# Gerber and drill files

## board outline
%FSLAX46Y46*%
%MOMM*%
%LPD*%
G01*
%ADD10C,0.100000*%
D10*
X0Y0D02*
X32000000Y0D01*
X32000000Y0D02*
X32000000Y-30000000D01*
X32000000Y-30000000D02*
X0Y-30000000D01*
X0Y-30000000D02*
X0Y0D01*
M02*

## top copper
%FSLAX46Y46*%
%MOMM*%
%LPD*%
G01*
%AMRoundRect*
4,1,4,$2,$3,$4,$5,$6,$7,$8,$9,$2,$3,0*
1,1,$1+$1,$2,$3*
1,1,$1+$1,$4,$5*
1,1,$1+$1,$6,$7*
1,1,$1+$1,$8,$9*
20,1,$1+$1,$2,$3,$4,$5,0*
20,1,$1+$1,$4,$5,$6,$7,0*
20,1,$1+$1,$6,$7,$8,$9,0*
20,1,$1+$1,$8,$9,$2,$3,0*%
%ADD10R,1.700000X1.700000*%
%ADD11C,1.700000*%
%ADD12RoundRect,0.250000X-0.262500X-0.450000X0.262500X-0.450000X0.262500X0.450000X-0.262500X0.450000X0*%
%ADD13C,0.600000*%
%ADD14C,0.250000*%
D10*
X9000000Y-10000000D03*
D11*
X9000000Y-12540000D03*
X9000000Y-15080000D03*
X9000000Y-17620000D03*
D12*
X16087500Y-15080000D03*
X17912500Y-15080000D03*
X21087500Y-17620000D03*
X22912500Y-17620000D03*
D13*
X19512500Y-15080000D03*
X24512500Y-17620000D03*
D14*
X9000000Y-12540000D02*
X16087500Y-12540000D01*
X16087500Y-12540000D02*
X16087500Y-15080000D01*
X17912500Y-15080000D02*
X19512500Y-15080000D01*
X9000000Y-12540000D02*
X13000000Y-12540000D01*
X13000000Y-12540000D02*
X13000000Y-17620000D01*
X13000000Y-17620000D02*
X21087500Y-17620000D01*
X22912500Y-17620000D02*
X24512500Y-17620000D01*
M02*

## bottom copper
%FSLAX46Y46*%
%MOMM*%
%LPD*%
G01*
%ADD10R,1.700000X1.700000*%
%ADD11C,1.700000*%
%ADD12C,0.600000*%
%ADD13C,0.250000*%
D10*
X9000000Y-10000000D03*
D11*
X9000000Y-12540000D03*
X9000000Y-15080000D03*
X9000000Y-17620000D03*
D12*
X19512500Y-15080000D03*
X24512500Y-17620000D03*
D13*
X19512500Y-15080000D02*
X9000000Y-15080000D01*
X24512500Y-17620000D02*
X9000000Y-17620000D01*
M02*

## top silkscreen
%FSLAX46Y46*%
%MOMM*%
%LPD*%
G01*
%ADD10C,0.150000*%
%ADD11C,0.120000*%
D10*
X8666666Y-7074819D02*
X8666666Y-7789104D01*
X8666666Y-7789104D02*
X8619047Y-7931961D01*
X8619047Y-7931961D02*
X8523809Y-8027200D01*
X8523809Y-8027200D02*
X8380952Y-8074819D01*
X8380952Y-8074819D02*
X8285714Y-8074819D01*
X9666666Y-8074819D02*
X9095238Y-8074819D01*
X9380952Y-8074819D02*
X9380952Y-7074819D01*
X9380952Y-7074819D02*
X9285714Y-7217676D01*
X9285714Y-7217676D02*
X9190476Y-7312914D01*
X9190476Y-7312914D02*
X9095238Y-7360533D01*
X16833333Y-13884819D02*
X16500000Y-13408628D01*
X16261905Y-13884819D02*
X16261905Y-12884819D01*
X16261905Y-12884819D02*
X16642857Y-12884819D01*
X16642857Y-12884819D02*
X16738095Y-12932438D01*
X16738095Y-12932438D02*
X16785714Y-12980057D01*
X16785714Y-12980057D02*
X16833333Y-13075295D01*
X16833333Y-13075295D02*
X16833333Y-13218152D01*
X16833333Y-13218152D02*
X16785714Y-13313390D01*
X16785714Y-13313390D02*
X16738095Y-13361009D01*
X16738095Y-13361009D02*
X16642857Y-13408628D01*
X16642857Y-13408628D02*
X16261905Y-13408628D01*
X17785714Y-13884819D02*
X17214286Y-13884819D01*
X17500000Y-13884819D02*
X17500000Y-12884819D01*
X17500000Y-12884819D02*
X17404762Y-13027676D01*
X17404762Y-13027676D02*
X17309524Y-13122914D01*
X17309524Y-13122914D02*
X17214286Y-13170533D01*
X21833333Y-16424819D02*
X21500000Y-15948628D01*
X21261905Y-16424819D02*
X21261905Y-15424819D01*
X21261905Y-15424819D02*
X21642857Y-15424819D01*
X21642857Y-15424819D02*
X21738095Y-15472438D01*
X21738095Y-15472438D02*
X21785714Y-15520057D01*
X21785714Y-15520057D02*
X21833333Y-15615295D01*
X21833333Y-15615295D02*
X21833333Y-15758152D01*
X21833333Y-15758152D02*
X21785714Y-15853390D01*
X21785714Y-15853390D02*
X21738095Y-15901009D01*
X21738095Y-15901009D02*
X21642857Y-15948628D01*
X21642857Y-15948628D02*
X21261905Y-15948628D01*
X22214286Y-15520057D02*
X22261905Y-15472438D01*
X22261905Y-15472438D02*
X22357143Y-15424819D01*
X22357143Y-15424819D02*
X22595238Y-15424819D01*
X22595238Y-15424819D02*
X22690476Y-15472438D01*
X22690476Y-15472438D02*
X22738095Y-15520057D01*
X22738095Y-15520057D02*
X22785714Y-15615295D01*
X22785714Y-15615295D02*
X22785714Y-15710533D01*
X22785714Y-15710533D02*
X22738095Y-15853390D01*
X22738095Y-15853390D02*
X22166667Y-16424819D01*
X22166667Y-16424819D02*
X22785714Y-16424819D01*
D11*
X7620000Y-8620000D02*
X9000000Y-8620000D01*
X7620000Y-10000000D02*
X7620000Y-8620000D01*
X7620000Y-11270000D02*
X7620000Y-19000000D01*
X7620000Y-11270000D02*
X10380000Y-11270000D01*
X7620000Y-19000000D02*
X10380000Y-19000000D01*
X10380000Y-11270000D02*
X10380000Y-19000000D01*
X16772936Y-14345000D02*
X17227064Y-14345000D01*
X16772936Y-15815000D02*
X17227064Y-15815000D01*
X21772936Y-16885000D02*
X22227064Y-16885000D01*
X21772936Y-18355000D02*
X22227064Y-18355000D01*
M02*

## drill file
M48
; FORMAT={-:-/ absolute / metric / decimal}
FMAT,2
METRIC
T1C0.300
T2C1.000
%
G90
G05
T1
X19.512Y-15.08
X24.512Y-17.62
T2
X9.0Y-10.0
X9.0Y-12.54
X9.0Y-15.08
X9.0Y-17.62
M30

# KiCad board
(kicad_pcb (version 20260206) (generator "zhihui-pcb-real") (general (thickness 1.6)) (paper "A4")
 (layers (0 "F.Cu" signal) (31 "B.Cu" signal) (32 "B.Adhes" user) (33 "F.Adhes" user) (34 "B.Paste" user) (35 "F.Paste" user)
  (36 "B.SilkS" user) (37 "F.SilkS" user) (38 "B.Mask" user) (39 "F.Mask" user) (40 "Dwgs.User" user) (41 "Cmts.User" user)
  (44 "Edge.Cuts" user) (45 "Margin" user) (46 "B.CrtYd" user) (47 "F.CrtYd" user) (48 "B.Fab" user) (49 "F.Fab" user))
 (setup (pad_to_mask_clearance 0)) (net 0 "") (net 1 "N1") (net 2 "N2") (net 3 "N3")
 (gr_line (start 0 0) (end 32 0) (stroke (width 0.1) (type default)) (layer "Edge.Cuts"))
 (gr_line (start 32 0) (end 32 30) (stroke (width 0.1) (type default)) (layer "Edge.Cuts"))
 (gr_line (start 32 30) (end 0 30) (stroke (width 0.1) (type default)) (layer "Edge.Cuts"))
 (gr_line (start 0 30) (end 0 0) (stroke (width 0.1) (type default)) (layer "Edge.Cuts"))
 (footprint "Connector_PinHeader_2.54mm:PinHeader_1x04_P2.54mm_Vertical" (layer "F.Cu")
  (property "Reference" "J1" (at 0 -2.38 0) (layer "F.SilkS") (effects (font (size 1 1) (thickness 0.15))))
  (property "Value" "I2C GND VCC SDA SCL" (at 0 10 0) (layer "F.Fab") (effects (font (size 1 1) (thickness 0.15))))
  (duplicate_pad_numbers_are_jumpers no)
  (fp_line (start -1.38 -1.38) (end 0 -1.38) (stroke (width 0.12) (type solid)) (layer "F.SilkS"))
  (fp_line (start -1.38 0) (end -1.38 -1.38) (stroke (width 0.12) (type solid)) (layer "F.SilkS"))
  (fp_line (start -1.38 1.27) (end -1.38 9) (stroke (width 0.12) (type solid)) (layer "F.SilkS"))
  (fp_line (start -1.38 1.27) (end 1.38 1.27) (stroke (width 0.12) (type solid)) (layer "F.SilkS"))
  (fp_line (start -1.38 9) (end 1.38 9) (stroke (width 0.12) (type solid)) (layer "F.SilkS"))
  (fp_line (start 1.38 1.27) (end 1.38 9) (stroke (width 0.12) (type solid)) (layer "F.SilkS"))
  (pad "1" thru_hole rect (at 0 0) (size 1.7 1.7) (drill 1) (layers "*.Cu" "*.Mask") (remove_unused_layers no))
  (pad "2" thru_hole circle (at 0 2.54) (size 1.7 1.7) (drill 1) (layers "*.Cu" "*.Mask") (remove_unused_layers no) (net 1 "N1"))
  (pad "3" thru_hole circle (at 0 5.08) (size 1.7 1.7) (drill 1) (layers "*.Cu" "*.Mask") (remove_unused_layers no) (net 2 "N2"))
  (pad "4" thru_hole circle (at 0 7.62) (size 1.7 1.7) (drill 1) (layers "*.Cu" "*.Mask") (remove_unused_layers no) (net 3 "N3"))
  (at 9 10 0))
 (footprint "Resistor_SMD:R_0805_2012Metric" (layer "F.Cu")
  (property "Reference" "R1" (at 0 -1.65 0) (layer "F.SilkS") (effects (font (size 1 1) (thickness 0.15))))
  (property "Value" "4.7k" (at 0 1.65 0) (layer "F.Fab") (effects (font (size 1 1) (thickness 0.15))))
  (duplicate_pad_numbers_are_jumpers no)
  (fp_line (start -0.227064 -0.735) (end 0.227064 -0.735) (stroke (width 0.12) (type solid)) (layer "F.SilkS"))
  (fp_line (start -0.227064 0.735) (end 0.227064 0.735) (stroke (width 0.12) (type solid)) (layer "F.SilkS"))
  (pad "1" smd roundrect (at -0.9125 0) (size 1.025 1.4) (layers "F.Cu" "F.Mask" "F.Paste") (roundrect_rratio 0.243902) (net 1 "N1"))
  (pad "2" smd roundrect (at 0.9125 0) (size 1.025 1.4) (layers "F.Cu" "F.Mask" "F.Paste") (roundrect_rratio 0.243902) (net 2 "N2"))
  (at 17 15.08 0))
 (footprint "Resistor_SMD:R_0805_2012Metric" (layer "F.Cu")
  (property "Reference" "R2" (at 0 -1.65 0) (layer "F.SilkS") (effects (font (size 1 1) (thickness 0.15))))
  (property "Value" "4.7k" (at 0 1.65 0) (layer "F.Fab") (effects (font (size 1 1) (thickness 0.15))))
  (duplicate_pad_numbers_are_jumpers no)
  (fp_line (start -0.227064 -0.735) (end 0.227064 -0.735) (stroke (width 0.12) (type solid)) (layer "F.SilkS"))
  (fp_line (start -0.227064 0.735) (end 0.227064 0.735) (stroke (width 0.12) (type solid)) (layer "F.SilkS"))
  (pad "1" smd roundrect (at -0.9125 0) (size 1.025 1.4) (layers "F.Cu" "F.Mask" "F.Paste") (roundrect_rratio 0.243902) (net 1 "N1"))
  (pad "2" smd roundrect (at 0.9125 0) (size 1.025 1.4) (layers "F.Cu" "F.Mask" "F.Paste") (roundrect_rratio 0.243902) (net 3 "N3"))
  (at 22 17.62 0))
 (segment (start 9 12.54) (end 16.0875 12.54) (width 0.25) (layer "F.Cu") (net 1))
 (segment (start 16.0875 12.54) (end 16.0875 15.08) (width 0.25) (layer "F.Cu") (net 1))
 (segment (start 17.9125 15.08) (end 19.5125 15.08) (width 0.25) (layer "F.Cu") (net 2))
 (segment (start 19.5125 15.08) (end 9 15.08) (width 0.25) (layer "B.Cu") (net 2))
 (segment (start 9 12.54) (end 13 12.54) (width 0.25) (layer "F.Cu") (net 1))
 (segment (start 13 12.54) (end 13 17.62) (width 0.25) (layer "F.Cu") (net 1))
 (segment (start 13 17.62) (end 21.0875 17.62) (width 0.25) (layer "F.Cu") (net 1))
 (segment (start 22.9125 17.62) (end 24.5125 17.62) (width 0.25) (layer "F.Cu") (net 3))
 (segment (start 24.5125 17.62) (end 9 17.62) (width 0.25) (layer "B.Cu") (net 3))
 (via (at 19.5125 15.08) (size 0.6) (drill 0.3) (layers "F.Cu" "B.Cu") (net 2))
 (via (at 24.5125 17.62) (size 0.6) (drill 0.3) (layers "F.Cu" "B.Cu") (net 3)))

